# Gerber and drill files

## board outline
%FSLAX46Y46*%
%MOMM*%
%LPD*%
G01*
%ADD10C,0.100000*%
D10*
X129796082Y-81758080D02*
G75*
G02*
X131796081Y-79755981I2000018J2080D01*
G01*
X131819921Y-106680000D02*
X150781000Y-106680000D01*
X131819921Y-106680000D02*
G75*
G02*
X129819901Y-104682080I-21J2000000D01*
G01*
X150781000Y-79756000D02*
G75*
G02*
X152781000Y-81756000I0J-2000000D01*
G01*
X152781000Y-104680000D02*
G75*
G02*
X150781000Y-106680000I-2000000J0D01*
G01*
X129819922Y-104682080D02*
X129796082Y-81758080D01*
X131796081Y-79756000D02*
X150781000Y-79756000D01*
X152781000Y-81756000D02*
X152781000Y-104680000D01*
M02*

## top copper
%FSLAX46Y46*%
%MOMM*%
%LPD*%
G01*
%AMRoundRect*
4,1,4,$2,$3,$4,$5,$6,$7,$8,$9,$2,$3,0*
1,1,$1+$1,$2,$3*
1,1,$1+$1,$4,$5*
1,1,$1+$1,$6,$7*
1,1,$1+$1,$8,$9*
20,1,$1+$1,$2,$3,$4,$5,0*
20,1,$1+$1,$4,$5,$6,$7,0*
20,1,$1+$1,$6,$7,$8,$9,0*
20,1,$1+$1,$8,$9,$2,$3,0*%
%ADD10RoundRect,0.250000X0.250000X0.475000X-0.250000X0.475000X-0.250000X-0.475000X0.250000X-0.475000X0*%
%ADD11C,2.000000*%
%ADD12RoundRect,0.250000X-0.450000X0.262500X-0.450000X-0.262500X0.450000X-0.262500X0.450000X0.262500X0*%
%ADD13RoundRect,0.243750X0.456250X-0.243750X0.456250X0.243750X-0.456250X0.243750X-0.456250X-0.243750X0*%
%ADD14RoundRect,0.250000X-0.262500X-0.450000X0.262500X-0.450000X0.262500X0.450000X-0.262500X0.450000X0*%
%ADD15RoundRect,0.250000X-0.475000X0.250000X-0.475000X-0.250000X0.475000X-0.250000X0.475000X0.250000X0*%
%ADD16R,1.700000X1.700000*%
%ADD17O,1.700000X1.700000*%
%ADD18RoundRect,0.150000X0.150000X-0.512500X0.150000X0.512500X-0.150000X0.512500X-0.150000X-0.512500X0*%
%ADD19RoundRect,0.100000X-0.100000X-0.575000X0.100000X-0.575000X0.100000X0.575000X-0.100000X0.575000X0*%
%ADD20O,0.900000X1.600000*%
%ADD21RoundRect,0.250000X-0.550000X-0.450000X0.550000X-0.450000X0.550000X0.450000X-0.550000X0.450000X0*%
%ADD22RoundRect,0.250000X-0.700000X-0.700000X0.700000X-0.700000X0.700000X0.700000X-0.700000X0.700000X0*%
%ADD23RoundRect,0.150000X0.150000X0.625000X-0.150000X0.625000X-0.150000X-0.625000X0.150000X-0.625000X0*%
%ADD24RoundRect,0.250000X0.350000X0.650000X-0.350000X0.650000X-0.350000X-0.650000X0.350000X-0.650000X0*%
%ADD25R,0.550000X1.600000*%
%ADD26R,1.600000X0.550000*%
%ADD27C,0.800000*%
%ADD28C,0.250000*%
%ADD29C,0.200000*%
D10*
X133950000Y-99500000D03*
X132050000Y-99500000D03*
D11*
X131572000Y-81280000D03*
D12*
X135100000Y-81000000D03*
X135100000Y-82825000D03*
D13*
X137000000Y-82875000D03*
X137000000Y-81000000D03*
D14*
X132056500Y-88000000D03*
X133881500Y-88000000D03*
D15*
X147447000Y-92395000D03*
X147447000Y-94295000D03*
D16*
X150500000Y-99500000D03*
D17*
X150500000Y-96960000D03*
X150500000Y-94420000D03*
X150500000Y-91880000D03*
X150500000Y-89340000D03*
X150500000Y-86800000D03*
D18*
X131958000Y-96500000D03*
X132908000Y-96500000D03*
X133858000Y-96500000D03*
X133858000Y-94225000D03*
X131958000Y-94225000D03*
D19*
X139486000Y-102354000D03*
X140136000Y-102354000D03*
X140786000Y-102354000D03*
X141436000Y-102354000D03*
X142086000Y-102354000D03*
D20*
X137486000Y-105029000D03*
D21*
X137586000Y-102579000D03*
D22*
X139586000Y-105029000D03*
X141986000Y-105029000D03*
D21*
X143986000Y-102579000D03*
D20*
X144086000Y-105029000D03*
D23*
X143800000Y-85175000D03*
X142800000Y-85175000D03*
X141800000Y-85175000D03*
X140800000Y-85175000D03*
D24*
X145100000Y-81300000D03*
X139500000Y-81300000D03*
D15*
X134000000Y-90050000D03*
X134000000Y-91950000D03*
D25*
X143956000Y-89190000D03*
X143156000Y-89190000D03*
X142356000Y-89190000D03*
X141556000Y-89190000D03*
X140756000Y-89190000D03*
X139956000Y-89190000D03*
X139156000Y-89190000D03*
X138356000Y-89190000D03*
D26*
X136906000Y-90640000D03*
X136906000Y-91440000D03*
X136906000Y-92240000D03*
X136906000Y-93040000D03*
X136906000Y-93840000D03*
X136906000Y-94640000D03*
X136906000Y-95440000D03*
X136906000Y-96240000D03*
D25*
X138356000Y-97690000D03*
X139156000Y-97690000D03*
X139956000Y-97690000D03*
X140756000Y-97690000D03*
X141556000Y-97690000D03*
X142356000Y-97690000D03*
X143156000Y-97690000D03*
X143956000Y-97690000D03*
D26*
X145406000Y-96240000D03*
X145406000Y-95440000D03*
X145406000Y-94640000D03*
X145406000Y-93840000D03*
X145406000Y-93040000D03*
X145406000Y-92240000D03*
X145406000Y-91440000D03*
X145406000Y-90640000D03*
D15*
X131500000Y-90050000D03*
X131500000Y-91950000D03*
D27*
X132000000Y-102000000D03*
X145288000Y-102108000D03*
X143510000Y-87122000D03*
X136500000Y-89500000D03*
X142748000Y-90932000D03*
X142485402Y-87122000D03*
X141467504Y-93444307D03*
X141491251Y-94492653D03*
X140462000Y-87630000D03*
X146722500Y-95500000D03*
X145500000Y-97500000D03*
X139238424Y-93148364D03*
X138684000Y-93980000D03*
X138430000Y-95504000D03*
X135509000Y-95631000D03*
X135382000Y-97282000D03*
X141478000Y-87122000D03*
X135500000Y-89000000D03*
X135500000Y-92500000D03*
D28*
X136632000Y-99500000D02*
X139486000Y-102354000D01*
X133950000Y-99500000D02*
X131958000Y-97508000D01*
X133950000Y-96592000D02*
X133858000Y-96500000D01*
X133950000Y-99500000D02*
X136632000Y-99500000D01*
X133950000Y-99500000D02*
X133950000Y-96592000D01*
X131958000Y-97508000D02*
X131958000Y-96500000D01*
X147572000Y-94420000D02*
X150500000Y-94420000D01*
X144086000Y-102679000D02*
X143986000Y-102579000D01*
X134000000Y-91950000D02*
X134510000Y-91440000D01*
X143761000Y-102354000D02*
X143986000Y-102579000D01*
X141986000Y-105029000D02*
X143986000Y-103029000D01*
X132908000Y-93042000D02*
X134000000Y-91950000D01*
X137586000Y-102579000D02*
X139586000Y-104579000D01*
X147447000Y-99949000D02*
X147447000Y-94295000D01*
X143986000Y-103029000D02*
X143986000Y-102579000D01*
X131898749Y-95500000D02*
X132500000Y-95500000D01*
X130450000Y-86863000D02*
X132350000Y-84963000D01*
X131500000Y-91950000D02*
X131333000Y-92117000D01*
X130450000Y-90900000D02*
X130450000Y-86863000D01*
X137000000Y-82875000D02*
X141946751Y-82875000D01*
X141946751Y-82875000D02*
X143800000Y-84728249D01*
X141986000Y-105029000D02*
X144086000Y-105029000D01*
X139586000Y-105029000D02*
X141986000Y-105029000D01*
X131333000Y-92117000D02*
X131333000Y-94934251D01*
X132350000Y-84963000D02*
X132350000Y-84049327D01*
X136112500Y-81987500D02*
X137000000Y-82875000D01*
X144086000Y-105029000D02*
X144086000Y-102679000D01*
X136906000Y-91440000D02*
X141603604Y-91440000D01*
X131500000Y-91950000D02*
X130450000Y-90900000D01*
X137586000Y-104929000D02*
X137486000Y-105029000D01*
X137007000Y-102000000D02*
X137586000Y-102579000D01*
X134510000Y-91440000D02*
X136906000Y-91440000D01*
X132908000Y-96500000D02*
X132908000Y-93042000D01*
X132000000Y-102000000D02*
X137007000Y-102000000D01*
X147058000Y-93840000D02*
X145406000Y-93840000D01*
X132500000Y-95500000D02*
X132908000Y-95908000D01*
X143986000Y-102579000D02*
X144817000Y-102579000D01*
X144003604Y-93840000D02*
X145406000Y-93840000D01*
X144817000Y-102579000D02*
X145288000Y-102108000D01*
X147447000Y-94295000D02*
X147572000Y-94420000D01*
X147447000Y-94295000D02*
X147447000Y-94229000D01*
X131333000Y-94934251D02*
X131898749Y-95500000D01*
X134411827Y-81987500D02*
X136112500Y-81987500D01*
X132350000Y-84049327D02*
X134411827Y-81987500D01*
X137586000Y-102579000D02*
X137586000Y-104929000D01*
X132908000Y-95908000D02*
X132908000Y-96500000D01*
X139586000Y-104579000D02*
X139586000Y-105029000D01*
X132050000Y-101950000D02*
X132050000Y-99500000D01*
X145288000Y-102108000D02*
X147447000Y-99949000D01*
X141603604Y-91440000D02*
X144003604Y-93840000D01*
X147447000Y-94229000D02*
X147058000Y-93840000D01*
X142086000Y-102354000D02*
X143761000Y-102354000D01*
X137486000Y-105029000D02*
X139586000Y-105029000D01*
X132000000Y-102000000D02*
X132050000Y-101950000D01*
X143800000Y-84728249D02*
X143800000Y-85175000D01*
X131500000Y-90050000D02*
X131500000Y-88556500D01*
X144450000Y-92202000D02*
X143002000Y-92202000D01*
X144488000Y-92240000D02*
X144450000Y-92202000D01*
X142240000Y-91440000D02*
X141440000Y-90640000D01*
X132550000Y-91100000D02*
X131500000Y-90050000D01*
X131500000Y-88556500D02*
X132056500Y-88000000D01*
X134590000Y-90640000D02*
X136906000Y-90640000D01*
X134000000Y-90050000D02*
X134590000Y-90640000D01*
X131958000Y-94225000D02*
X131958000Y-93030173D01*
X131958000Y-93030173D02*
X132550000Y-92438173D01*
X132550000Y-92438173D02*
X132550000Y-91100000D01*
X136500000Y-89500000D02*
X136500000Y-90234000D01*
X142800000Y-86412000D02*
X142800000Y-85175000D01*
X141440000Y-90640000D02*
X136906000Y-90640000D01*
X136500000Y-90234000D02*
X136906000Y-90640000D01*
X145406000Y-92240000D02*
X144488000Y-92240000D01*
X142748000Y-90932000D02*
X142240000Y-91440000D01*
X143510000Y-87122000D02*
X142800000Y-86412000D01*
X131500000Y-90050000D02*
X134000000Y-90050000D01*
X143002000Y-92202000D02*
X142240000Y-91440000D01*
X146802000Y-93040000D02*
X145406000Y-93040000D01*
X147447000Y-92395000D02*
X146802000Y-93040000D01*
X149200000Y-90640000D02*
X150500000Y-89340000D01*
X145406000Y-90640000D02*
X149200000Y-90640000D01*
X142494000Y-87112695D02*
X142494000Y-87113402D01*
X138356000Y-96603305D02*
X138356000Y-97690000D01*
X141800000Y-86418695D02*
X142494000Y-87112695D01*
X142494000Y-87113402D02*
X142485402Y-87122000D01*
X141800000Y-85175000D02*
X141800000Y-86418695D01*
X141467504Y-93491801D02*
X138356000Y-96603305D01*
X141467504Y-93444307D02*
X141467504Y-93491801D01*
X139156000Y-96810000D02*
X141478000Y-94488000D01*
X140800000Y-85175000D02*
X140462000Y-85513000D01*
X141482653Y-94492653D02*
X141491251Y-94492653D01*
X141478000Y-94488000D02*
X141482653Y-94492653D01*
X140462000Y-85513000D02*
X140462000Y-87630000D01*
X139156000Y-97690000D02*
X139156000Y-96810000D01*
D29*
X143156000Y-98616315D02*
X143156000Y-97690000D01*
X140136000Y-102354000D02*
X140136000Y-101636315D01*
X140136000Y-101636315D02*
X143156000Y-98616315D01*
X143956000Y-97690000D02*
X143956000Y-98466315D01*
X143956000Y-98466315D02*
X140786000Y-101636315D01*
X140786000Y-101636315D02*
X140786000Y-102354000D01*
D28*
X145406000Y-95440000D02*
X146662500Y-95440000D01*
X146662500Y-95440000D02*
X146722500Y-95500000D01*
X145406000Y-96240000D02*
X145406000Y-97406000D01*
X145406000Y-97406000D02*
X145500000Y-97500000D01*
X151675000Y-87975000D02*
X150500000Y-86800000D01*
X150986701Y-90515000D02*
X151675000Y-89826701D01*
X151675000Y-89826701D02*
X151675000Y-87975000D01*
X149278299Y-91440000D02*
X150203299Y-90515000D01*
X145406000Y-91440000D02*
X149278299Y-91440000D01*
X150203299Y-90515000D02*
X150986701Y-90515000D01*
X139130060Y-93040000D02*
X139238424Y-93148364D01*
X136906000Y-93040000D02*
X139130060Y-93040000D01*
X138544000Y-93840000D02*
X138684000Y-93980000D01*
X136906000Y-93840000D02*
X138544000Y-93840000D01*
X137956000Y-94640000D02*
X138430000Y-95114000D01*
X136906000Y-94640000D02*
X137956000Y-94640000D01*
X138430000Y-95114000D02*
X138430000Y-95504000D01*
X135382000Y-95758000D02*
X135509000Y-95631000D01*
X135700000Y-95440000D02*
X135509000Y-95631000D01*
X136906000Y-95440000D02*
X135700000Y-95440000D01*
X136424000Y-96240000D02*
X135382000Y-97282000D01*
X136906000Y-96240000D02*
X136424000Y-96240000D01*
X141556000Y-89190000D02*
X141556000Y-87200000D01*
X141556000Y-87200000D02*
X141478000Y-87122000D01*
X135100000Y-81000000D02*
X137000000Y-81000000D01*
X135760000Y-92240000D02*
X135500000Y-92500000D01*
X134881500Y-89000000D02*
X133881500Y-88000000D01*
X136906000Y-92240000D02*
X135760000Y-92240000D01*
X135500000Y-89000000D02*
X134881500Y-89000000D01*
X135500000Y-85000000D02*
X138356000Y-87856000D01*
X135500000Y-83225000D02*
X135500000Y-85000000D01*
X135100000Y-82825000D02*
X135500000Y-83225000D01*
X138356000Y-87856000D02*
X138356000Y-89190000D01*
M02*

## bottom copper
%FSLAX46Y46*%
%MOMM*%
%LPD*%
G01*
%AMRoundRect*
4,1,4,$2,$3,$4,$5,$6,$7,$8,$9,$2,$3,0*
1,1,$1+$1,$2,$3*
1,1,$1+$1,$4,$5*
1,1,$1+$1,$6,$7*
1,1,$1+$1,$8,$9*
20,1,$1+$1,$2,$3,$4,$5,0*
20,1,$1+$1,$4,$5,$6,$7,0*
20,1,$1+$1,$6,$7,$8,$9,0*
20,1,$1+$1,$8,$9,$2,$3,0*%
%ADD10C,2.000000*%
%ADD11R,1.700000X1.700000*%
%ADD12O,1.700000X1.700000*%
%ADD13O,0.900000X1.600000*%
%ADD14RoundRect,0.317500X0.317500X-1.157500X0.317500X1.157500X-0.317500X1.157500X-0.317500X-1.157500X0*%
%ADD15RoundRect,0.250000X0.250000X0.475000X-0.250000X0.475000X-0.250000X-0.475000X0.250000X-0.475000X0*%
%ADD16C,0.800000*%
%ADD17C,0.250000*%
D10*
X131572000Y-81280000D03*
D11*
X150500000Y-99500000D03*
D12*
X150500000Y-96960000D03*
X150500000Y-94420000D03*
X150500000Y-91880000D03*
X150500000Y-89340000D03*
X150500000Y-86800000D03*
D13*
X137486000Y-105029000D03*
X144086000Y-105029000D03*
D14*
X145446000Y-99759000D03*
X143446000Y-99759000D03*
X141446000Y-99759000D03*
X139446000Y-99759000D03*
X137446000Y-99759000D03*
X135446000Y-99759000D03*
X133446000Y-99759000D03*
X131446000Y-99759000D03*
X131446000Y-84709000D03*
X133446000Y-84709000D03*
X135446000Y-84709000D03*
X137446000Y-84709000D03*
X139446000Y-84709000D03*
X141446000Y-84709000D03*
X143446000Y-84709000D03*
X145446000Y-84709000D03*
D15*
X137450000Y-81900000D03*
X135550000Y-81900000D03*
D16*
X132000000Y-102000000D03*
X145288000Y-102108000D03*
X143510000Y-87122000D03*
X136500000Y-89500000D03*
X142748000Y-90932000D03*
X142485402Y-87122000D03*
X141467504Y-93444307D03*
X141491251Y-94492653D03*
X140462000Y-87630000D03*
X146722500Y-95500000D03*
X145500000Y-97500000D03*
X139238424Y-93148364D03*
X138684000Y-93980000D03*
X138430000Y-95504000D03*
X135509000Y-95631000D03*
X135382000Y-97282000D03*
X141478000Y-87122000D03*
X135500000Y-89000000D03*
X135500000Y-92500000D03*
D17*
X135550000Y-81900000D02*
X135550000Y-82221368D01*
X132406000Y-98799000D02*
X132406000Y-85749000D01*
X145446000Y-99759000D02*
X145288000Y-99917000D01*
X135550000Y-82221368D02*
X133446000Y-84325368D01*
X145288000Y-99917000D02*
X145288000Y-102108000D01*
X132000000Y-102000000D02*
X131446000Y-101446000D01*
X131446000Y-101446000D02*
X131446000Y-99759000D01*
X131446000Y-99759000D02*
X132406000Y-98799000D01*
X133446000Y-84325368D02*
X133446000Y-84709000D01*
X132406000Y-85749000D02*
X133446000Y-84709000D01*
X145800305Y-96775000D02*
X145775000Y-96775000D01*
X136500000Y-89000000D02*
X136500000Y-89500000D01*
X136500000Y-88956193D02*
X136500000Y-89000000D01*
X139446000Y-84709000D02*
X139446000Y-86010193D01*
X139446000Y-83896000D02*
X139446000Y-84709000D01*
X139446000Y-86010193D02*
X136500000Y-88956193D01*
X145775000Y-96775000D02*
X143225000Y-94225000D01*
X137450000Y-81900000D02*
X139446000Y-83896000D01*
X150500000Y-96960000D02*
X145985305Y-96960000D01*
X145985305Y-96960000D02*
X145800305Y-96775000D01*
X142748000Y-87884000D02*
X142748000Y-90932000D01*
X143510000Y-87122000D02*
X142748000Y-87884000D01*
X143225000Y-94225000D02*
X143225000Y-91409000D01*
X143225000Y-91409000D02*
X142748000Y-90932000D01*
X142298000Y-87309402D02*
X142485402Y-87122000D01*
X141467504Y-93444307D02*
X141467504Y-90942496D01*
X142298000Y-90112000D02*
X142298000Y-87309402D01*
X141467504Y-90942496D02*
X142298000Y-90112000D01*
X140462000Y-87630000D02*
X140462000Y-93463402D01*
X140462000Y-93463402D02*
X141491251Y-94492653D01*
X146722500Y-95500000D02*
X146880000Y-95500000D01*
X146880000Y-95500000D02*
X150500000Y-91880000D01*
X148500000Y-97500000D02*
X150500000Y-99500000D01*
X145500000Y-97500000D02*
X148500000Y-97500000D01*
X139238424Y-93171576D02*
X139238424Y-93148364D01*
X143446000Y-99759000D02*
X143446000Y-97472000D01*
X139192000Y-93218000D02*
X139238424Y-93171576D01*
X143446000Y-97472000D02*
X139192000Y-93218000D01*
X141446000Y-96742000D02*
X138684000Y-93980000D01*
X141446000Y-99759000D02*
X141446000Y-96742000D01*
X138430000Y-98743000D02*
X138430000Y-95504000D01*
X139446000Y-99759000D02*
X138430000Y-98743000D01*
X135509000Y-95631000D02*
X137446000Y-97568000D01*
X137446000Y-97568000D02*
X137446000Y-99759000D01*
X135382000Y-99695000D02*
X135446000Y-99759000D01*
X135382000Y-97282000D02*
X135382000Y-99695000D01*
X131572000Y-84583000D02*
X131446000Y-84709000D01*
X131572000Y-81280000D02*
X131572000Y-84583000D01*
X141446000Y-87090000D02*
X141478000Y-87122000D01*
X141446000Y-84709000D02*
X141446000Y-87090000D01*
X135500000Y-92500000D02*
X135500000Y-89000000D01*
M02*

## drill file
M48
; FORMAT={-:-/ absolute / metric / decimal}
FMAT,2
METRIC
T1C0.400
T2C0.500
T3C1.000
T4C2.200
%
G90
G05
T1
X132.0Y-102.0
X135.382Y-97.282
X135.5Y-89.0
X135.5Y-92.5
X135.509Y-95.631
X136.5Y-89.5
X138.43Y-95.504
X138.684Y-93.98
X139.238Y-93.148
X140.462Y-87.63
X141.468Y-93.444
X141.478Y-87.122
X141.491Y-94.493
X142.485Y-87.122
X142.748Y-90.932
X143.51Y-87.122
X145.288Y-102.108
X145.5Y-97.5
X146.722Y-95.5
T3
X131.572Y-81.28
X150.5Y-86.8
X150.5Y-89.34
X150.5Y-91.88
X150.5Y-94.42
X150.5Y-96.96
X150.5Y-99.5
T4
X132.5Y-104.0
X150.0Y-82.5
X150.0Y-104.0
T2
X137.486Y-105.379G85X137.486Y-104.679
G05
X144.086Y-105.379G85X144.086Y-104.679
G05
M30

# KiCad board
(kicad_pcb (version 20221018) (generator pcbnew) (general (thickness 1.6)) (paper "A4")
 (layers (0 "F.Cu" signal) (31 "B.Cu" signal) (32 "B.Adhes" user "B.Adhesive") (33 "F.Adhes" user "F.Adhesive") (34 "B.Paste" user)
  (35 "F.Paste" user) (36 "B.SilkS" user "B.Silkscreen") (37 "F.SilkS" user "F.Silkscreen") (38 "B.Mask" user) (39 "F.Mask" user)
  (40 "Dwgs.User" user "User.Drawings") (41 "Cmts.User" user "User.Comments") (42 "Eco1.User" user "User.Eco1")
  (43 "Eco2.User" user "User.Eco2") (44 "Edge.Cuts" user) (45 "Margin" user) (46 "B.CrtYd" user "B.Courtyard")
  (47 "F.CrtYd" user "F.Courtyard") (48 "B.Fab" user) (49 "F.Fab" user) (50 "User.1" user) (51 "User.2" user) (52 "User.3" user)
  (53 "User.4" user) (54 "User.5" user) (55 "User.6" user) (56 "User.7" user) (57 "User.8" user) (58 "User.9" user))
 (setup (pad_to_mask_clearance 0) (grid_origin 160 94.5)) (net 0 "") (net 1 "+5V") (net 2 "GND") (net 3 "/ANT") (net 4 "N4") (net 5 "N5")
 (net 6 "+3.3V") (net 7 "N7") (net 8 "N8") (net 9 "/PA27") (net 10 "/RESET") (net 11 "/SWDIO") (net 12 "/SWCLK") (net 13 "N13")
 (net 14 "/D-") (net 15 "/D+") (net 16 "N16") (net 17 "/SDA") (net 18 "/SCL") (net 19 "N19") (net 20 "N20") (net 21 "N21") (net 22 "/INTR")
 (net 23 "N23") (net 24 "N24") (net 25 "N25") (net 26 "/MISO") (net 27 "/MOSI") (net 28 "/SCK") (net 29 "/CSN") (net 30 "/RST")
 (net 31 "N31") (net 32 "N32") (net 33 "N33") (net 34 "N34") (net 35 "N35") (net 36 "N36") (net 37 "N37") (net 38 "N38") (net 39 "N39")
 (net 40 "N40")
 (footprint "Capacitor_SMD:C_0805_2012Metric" (layer "F.Cu") (at 133 99.5 180)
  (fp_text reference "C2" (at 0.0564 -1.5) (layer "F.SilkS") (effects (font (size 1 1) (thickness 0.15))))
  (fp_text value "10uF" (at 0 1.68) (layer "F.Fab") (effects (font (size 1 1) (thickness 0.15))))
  (pad "1" smd roundrect (at -0.95 0 180) (size 1 1.45) (layers "F.Cu" "F.Paste" "F.Mask") (roundrect_rratio 0.25) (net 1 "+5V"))
  (pad "2" smd roundrect (at 0.95 0 180) (size 1 1.45) (layers "F.Cu" "F.Paste" "F.Mask") (roundrect_rratio 0.25) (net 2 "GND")))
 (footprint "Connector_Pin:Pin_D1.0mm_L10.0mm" (layer "F.Cu") (at 131.572 81.28)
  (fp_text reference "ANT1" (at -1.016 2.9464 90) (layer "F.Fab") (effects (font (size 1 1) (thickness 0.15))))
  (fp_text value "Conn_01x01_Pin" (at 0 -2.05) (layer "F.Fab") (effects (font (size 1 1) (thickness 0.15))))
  (pad "1" thru_hole circle (at 0 0) (size 2 2) (drill 1) (layers "*.Cu" "*.Mask") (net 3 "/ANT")))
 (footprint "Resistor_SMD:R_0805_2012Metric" (layer "F.Cu") (at 135.1 81.9125 -90)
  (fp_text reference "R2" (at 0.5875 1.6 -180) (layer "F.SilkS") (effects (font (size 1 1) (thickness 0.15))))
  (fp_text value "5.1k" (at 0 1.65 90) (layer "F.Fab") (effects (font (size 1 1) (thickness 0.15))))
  (pad "1" smd roundrect (at -0.9125 0 270) (size 1.025 1.4) (layers "F.Cu" "F.Paste" "F.Mask") (roundrect_rratio 0.243902) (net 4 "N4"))
  (pad "2" smd roundrect (at 0.9125 0 270) (size 1.025 1.4) (layers "F.Cu" "F.Paste" "F.Mask") (roundrect_rratio 0.243902) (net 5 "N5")))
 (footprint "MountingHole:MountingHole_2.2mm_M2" (layer "F.Cu") (at 150 104)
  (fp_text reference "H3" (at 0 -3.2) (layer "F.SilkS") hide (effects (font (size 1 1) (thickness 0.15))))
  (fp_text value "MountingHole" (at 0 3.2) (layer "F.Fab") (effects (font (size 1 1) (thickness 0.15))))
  (pad "" np_thru_hole circle (at 0 0) (size 2.2 2.2) (drill 2.2) (layers "*.Cu" "*.Mask")))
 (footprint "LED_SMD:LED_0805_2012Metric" (layer "F.Cu") (at 137 81.9375 90)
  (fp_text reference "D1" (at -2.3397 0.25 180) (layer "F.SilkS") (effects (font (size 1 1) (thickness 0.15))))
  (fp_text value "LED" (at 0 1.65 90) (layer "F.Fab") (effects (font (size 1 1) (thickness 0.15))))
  (pad "1" smd roundrect (at -0.9375 0 90) (size 0.975 1.4) (layers "F.Cu" "F.Paste" "F.Mask") (roundrect_rratio 0.25) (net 2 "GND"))
  (pad "2" smd roundrect (at 0.9375 0 90) (size 0.975 1.4) (layers "F.Cu" "F.Paste" "F.Mask") (roundrect_rratio 0.25) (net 4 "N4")))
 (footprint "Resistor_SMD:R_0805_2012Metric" (layer "F.Cu") (at 132.969 88)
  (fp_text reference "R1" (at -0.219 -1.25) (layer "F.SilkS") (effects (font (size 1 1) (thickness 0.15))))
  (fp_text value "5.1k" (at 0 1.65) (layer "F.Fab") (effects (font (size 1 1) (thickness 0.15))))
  (pad "1" smd roundrect (at -0.9125 0) (size 1.025 1.4) (layers "F.Cu" "F.Paste" "F.Mask") (roundrect_rratio 0.243902) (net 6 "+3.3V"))
  (pad "2" smd roundrect (at 0.9125 0) (size 1.025 1.4) (layers "F.Cu" "F.Paste" "F.Mask") (roundrect_rratio 0.243902) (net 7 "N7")))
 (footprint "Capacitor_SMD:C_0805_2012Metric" (layer "F.Cu") (at 147.447 93.345 -90)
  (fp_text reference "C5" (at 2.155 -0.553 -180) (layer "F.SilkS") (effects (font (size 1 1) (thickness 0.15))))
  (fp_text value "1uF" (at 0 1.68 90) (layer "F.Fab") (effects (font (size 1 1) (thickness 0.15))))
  (pad "1" smd roundrect (at -0.95 0 270) (size 1 1.45) (layers "F.Cu" "F.Paste" "F.Mask") (roundrect_rratio 0.25) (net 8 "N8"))
  (pad "2" smd roundrect (at 0.95 0 270) (size 1 1.45) (layers "F.Cu" "F.Paste" "F.Mask") (roundrect_rratio 0.25) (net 2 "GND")))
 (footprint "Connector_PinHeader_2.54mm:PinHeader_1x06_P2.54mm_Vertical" (layer "F.Cu") (at 150.5 99.5 180)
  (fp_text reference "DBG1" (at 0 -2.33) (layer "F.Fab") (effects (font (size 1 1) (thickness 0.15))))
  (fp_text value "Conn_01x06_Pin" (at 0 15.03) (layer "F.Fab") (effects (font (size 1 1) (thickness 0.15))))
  (pad "1" thru_hole rect (at 0 0 180) (size 1.7 1.7) (drill 1) (layers "*.Cu" "*.Mask") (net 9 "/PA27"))
  (pad "2" thru_hole oval (at 0 2.54 180) (size 1.7 1.7) (drill 1) (layers "*.Cu" "*.Mask") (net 6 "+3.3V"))
  (pad "3" thru_hole oval (at 0 5.08 180) (size 1.7 1.7) (drill 1) (layers "*.Cu" "*.Mask") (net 2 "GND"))
  (pad "4" thru_hole oval (at 0 7.62 180) (size 1.7 1.7) (drill 1) (layers "*.Cu" "*.Mask") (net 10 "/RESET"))
  (pad "5" thru_hole oval (at 0 10.16 180) (size 1.7 1.7) (drill 1) (layers "*.Cu" "*.Mask") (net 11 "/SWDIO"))
  (pad "6" thru_hole oval (at 0 12.7 180) (size 1.7 1.7) (drill 1) (layers "*.Cu" "*.Mask") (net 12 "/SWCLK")))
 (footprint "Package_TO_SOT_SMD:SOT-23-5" (layer "F.Cu") (at 132.908 95.3625 90)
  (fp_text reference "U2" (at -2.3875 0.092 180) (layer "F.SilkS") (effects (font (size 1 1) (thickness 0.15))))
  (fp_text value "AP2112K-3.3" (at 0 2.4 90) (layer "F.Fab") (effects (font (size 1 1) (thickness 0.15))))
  (pad "1" smd roundrect (at -1.1375 -0.95 90) (size 1.325 0.6) (layers "F.Cu" "F.Paste" "F.Mask") (roundrect_rratio 0.25) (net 1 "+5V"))
  (pad "2" smd roundrect (at -1.1375 0 90) (size 1.325 0.6) (layers "F.Cu" "F.Paste" "F.Mask") (roundrect_rratio 0.25) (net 2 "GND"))
  (pad "3" smd roundrect (at -1.1375 0.95 90) (size 1.325 0.6) (layers "F.Cu" "F.Paste" "F.Mask") (roundrect_rratio 0.25) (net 1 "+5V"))
  (pad "4" smd roundrect (at 1.1375 0.95 90) (size 1.325 0.6) (layers "F.Cu" "F.Paste" "F.Mask") (roundrect_rratio 0.25) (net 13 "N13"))
  (pad "5" smd roundrect (at 1.1375 -0.95 90) (size 1.325 0.6) (layers "F.Cu" "F.Paste" "F.Mask") (roundrect_rratio 0.25) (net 6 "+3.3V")))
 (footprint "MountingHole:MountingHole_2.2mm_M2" (layer "F.Cu") (at 150 82.5)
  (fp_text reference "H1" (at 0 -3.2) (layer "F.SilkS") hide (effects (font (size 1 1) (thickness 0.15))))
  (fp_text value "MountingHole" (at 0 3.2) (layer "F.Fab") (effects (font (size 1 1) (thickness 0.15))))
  (pad "" np_thru_hole circle (at 0 0) (size 2.2 2.2) (drill 2.2) (layers "*.Cu" "*.Mask")))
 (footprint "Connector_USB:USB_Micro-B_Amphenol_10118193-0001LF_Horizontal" (layer "F.Cu") (at 140.786 105.029)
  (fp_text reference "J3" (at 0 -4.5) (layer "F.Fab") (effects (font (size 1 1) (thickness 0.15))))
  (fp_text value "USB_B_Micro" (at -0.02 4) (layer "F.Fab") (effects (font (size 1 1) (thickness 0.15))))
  (pad "1" smd roundrect (at -1.3 -2.675) (size 0.4 1.35) (layers "F.Cu" "F.Paste" "F.Mask") (roundrect_rratio 0.25) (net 1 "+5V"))
  (pad "2" smd roundrect (at -0.65 -2.675) (size 0.4 1.35) (layers "F.Cu" "F.Paste" "F.Mask") (roundrect_rratio 0.25) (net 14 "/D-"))
  (pad "3" smd roundrect (at 0 -2.675) (size 0.4 1.35) (layers "F.Cu" "F.Paste" "F.Mask") (roundrect_rratio 0.25) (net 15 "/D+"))
  (pad "4" smd roundrect (at 0.65 -2.675) (size 0.4 1.35) (layers "F.Cu" "F.Paste" "F.Mask") (roundrect_rratio 0.25) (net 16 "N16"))
  (pad "5" smd roundrect (at 1.3 -2.675) (size 0.4 1.35) (layers "F.Cu" "F.Paste" "F.Mask") (roundrect_rratio 0.25) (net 2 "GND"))
  (pad "6" thru_hole oval (at -3.3 0 90) (size 1.6 0.9) (drill oval 1.2 0.5) (layers "*.Cu" "*.Mask" "F.Paste") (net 2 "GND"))
  (pad "6" smd roundrect (at -3.2 -2.45) (size 1.6 1.4) (layers "F.Cu" "F.Paste" "F.Mask") (roundrect_rratio 0.1785714286) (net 2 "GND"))
  (pad "6" smd roundrect (at -1.2 0) (size 1.9 1.9) (layers "F.Cu" "F.Paste" "F.Mask") (roundrect_rratio 0.1315789474) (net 2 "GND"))
  (pad "6" smd roundrect (at 1.2 0) (size 1.9 1.9) (layers "F.Cu" "F.Paste" "F.Mask") (roundrect_rratio 0.1315789474) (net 2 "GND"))
  (pad "6" smd roundrect (at 3.2 -2.45) (size 1.6 1.4) (layers "F.Cu" "F.Paste" "F.Mask") (roundrect_rratio 0.1785714286) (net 2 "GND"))
  (pad "6" thru_hole oval (at 3.3 0 90) (size 1.6 0.9) (drill oval 1.2 0.5) (layers "*.Cu" "*.Mask" "F.Paste") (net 2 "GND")))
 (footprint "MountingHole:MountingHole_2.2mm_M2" (layer "F.Cu") (at 132.5 104)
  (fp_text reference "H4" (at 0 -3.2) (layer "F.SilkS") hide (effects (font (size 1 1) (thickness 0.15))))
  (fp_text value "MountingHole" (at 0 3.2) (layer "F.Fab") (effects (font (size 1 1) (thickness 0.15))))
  (pad "" np_thru_hole circle (at 0 0) (size 2.2 2.2) (drill 2.2) (layers "*.Cu" "*.Mask")))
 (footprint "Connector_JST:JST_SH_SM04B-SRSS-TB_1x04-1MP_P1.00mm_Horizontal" (layer "F.Cu") (at 142.3 83.175 180)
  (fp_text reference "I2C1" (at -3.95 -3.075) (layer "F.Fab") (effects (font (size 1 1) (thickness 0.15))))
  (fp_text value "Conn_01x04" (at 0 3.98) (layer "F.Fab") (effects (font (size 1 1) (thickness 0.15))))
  (pad "1" smd roundrect (at -1.5 -2 180) (size 0.6 1.55) (layers "F.Cu" "F.Paste" "F.Mask") (roundrect_rratio 0.25) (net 2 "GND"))
  (pad "2" smd roundrect (at -0.5 -2 180) (size 0.6 1.55) (layers "F.Cu" "F.Paste" "F.Mask") (roundrect_rratio 0.25) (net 6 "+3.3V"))
  (pad "3" smd roundrect (at 0.5 -2 180) (size 0.6 1.55) (layers "F.Cu" "F.Paste" "F.Mask") (roundrect_rratio 0.25) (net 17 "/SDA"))
  (pad "4" smd roundrect (at 1.5 -2 180) (size 0.6 1.55) (layers "F.Cu" "F.Paste" "F.Mask") (roundrect_rratio 0.25) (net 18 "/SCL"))
  (pad "MP" smd roundrect (at -2.8 1.875 180) (size 1.2 1.8) (layers "F.Cu" "F.Paste" "F.Mask") (roundrect_rratio 0.208333))
  (pad "MP" smd roundrect (at 2.8 1.875 180) (size 1.2 1.8) (layers "F.Cu" "F.Paste" "F.Mask") (roundrect_rratio 0.208333)))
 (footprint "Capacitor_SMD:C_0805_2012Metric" (layer "F.Cu") (at 134 91 -90)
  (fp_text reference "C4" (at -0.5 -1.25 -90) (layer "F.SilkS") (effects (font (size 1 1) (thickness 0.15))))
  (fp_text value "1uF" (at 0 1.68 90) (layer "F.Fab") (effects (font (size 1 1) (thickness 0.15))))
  (pad "1" smd roundrect (at -0.95 0 270) (size 1 1.45) (layers "F.Cu" "F.Paste" "F.Mask") (roundrect_rratio 0.25) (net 6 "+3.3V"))
  (pad "2" smd roundrect (at 0.95 0 270) (size 1 1.45) (layers "F.Cu" "F.Paste" "F.Mask") (roundrect_rratio 0.25) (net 2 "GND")))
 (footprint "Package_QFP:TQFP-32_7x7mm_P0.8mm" (layer "F.Cu") (at 141.156 93.44 -90)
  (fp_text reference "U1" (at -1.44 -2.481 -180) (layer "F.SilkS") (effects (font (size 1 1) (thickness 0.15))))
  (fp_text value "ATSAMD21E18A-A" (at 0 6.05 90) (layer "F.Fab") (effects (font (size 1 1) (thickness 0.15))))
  (pad "1" smd rect (at -4.25 -2.8 270) (size 1.6 0.55) (layers "F.Cu" "F.Paste" "F.Mask") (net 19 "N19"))
  (pad "2" smd rect (at -4.25 -2 270) (size 1.6 0.55) (layers "F.Cu" "F.Paste" "F.Mask") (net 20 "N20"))
  (pad "3" smd rect (at -4.25 -1.2 270) (size 1.6 0.55) (layers "F.Cu" "F.Paste" "F.Mask") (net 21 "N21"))
  (pad "4" smd rect (at -4.25 -0.4 270) (size 1.6 0.55) (layers "F.Cu" "F.Paste" "F.Mask") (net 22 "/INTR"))
  (pad "5" smd rect (at -4.25 0.4 270) (size 1.6 0.55) (layers "F.Cu" "F.Paste" "F.Mask") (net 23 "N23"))
  (pad "6" smd rect (at -4.25 1.2 270) (size 1.6 0.55) (layers "F.Cu" "F.Paste" "F.Mask") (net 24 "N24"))
  (pad "7" smd rect (at -4.25 2 270) (size 1.6 0.55) (layers "F.Cu" "F.Paste" "F.Mask") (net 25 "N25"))
  (pad "8" smd rect (at -4.25 2.8 270) (size 1.6 0.55) (layers "F.Cu" "F.Paste" "F.Mask") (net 5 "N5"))
  (pad "9" smd rect (at -2.8 4.25) (size 1.6 0.55) (layers "F.Cu" "F.Paste" "F.Mask") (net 6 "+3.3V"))
  (pad "10" smd rect (at -2 4.25) (size 1.6 0.55) (layers "F.Cu" "F.Paste" "F.Mask") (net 2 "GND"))
  (pad "11" smd rect (at -1.2 4.25) (size 1.6 0.55) (layers "F.Cu" "F.Paste" "F.Mask") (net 7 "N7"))
  (pad "12" smd rect (at -0.4 4.25) (size 1.6 0.55) (layers "F.Cu" "F.Paste" "F.Mask") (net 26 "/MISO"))
  (pad "13" smd rect (at 0.4 4.25) (size 1.6 0.55) (layers "F.Cu" "F.Paste" "F.Mask") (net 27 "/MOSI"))
  (pad "14" smd rect (at 1.2 4.25) (size 1.6 0.55) (layers "F.Cu" "F.Paste" "F.Mask") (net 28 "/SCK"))
  (pad "15" smd rect (at 2 4.25) (size 1.6 0.55) (layers "F.Cu" "F.Paste" "F.Mask") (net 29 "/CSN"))
  (pad "16" smd rect (at 2.8 4.25) (size 1.6 0.55) (layers "F.Cu" "F.Paste" "F.Mask") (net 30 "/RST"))
  (pad "17" smd rect (at 4.25 2.8 270) (size 1.6 0.55) (layers "F.Cu" "F.Paste" "F.Mask") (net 17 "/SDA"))
  (pad "18" smd rect (at 4.25 2 270) (size 1.6 0.55) (layers "F.Cu" "F.Paste" "F.Mask") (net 18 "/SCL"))
  (pad "19" smd rect (at 4.25 1.2 270) (size 1.6 0.55) (layers "F.Cu" "F.Paste" "F.Mask") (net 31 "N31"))
  (pad "20" smd rect (at 4.25 0.4 270) (size 1.6 0.55) (layers "F.Cu" "F.Paste" "F.Mask") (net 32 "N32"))
  (pad "21" smd rect (at 4.25 -0.4 270) (size 1.6 0.55) (layers "F.Cu" "F.Paste" "F.Mask") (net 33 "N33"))
  (pad "22" smd rect (at 4.25 -1.2 270) (size 1.6 0.55) (layers "F.Cu" "F.Paste" "F.Mask") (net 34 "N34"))
  (pad "23" smd rect (at 4.25 -2 270) (size 1.6 0.55) (layers "F.Cu" "F.Paste" "F.Mask") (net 14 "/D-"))
  (pad "24" smd rect (at 4.25 -2.8 270) (size 1.6 0.55) (layers "F.Cu" "F.Paste" "F.Mask") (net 15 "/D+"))
  (pad "25" smd rect (at 2.8 -4.25) (size 1.6 0.55) (layers "F.Cu" "F.Paste" "F.Mask") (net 9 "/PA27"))
  (pad "26" smd rect (at 2 -4.25) (size 1.6 0.55) (layers "F.Cu" "F.Paste" "F.Mask") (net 10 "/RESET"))
  (pad "27" smd rect (at 1.2 -4.25) (size 1.6 0.55) (layers "F.Cu" "F.Paste" "F.Mask") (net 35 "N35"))
  (pad "28" smd rect (at 0.4 -4.25) (size 1.6 0.55) (layers "F.Cu" "F.Paste" "F.Mask") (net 2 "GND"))
  (pad "29" smd rect (at -0.4 -4.25) (size 1.6 0.55) (layers "F.Cu" "F.Paste" "F.Mask") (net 8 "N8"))
  (pad "30" smd rect (at -1.2 -4.25) (size 1.6 0.55) (layers "F.Cu" "F.Paste" "F.Mask") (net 6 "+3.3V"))
  (pad "31" smd rect (at -2 -4.25) (size 1.6 0.55) (layers "F.Cu" "F.Paste" "F.Mask") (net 12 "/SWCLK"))
  (pad "32" smd rect (at -2.8 -4.25) (size 1.6 0.55) (layers "F.Cu" "F.Paste" "F.Mask") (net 11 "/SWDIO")))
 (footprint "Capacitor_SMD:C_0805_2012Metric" (layer "F.Cu") (at 131.5 91 -90)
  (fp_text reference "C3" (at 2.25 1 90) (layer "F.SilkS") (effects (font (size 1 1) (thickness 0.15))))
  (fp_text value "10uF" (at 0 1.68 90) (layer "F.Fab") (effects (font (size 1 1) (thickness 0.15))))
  (pad "1" smd roundrect (at -0.95 0 270) (size 1 1.45) (layers "F.Cu" "F.Paste" "F.Mask") (roundrect_rratio 0.25) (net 6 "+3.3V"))
  (pad "2" smd roundrect (at 0.95 0 270) (size 1 1.45) (layers "F.Cu" "F.Paste" "F.Mask") (roundrect_rratio 0.25) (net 2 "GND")))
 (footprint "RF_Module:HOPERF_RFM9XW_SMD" (layer "B.Cu") (at 138.446 92.234 90)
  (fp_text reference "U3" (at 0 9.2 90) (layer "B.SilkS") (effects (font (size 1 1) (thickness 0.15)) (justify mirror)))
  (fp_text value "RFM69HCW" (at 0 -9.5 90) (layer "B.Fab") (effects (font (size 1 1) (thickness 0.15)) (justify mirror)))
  (pad "1" smd roundrect (at -7.525 7 90) (size 2.95 1.27) (layers "B.Cu" "B.Paste" "B.Mask") (roundrect_rratio 0.25) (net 2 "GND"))
  (pad "2" smd roundrect (at -7.525 5 90) (size 2.95 1.27) (layers "B.Cu" "B.Paste" "B.Mask") (roundrect_rratio 0.25) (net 26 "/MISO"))
  (pad "3" smd roundrect (at -7.525 3 90) (size 2.95 1.27) (layers "B.Cu" "B.Paste" "B.Mask") (roundrect_rratio 0.25) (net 27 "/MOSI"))
  (pad "4" smd roundrect (at -7.525 1 90) (size 2.95 1.27) (layers "B.Cu" "B.Paste" "B.Mask") (roundrect_rratio 0.25) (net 28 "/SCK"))
  (pad "5" smd roundrect (at -7.525 -1 90) (size 2.95 1.27) (layers "B.Cu" "B.Paste" "B.Mask") (roundrect_rratio 0.25) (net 29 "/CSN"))
  (pad "6" smd roundrect (at -7.525 -3 90) (size 2.95 1.27) (layers "B.Cu" "B.Paste" "B.Mask") (roundrect_rratio 0.25) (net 30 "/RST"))
  (pad "7" smd roundrect (at -7.525 -5 90) (size 2.95 1.27) (layers "B.Cu" "B.Paste" "B.Mask") (roundrect_rratio 0.25) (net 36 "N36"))
  (pad "8" smd roundrect (at -7.525 -7 90) (size 2.95 1.27) (layers "B.Cu" "B.Paste" "B.Mask") (roundrect_rratio 0.25) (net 2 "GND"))
  (pad "9" smd roundrect (at 7.525 -7 90) (size 2.95 1.27) (layers "B.Cu" "B.Paste" "B.Mask") (roundrect_rratio 0.25) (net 3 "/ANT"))
  (pad "10" smd roundrect (at 7.525 -5 90) (size 2.95 1.27) (layers "B.Cu" "B.Paste" "B.Mask") (roundrect_rratio 0.25) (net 2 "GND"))
  (pad "11" smd roundrect (at 7.525 -3 90) (size 2.95 1.27) (layers "B.Cu" "B.Paste" "B.Mask") (roundrect_rratio 0.25) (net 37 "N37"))
  (pad "12" smd roundrect (at 7.525 -1 90) (size 2.95 1.27) (layers "B.Cu" "B.Paste" "B.Mask") (roundrect_rratio 0.25) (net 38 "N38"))
  (pad "13" smd roundrect (at 7.525 1 90) (size 2.95 1.27) (layers "B.Cu" "B.Paste" "B.Mask") (roundrect_rratio 0.25) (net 6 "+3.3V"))
  (pad "14" smd roundrect (at 7.525 3 90) (size 2.95 1.27) (layers "B.Cu" "B.Paste" "B.Mask") (roundrect_rratio 0.25) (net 22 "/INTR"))
  (pad "15" smd roundrect (at 7.525 5 90) (size 2.95 1.27) (layers "B.Cu" "B.Paste" "B.Mask") (roundrect_rratio 0.25) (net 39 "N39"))
  (pad "16" smd roundrect (at 7.525 7 90) (size 2.95 1.27) (layers "B.Cu" "B.Paste" "B.Mask") (roundrect_rratio 0.25) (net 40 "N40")))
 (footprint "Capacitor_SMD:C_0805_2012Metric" (layer "B.Cu") (at 136.5 81.9 180)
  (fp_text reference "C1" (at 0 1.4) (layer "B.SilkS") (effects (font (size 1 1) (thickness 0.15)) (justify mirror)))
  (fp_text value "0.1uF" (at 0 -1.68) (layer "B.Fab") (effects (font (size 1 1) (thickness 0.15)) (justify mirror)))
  (pad "1" smd roundrect (at -0.95 0 180) (size 1 1.45) (layers "B.Cu" "B.Paste" "B.Mask") (roundrect_rratio 0.25) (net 6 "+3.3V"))
  (pad "2" smd roundrect (at 0.95 0 180) (size 1 1.45) (layers "B.Cu" "B.Paste" "B.Mask") (roundrect_rratio 0.25) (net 2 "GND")))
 (gr_arc (start 129.796082 81.75808) (mid 130.381132 80.342522) (end 131.796081 79.756) (stroke (width 0.1) (type default))
  (layer "Edge.Cuts"))
 (gr_line (start 131.819921 106.68) (end 150.781 106.68) (stroke (width 0.1) (type default)) (layer "Edge.Cuts"))
 (gr_arc (start 131.819921 106.68) (mid 130.406443 106.094949) (end 129.819922 104.68208) (stroke (width 0.1) (type default))
  (layer "Edge.Cuts"))
 (gr_arc (start 150.781 79.756) (mid 152.195214 80.341786) (end 152.781 81.756) (stroke (width 0.1) (type default)) (layer "Edge.Cuts"))
 (gr_arc (start 152.781 104.68) (mid 152.195214 106.094214) (end 150.781 106.68) (stroke (width 0.1) (type default)) (layer "Edge.Cuts"))
 (gr_line (start 129.819922 104.68208) (end 129.796082 81.75808) (stroke (width 0.1) (type default)) (layer "Edge.Cuts"))
 (gr_line (start 131.796081 79.756) (end 150.781 79.756) (stroke (width 0.1) (type default)) (layer "Edge.Cuts"))
 (gr_line (start 152.781 81.756) (end 152.781 104.68) (stroke (width 0.1) (type default)) (layer "Edge.Cuts"))
 (segment (start 136.632 99.5) (end 139.486 102.354) (width 0.25) (layer "F.Cu") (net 1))
 (segment (start 133.95 99.5) (end 131.958 97.508) (width 0.25) (layer "F.Cu") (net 1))
 (segment (start 133.95 96.592) (end 133.858 96.5) (width 0.25) (layer "F.Cu") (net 1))
 (segment (start 133.95 99.5) (end 136.632 99.5) (width 0.25) (layer "F.Cu") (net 1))
 (segment (start 133.95 99.5) (end 133.95 96.592) (width 0.25) (layer "F.Cu") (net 1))
 (segment (start 131.958 97.508) (end 131.958 96.5) (width 0.25) (layer "F.Cu") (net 1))
 (segment (start 147.572 94.42) (end 150.5 94.42) (width 0.25) (layer "F.Cu") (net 2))
 (segment (start 144.086 102.679) (end 143.986 102.579) (width 0.25) (layer "F.Cu") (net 2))
 (segment (start 134 91.95) (end 134.51 91.44) (width 0.25) (layer "F.Cu") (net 2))
 (segment (start 143.761 102.354) (end 143.986 102.579) (width 0.25) (layer "F.Cu") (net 2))
 (segment (start 141.986 105.029) (end 143.986 103.029) (width 0.25) (layer "F.Cu") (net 2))
 (segment (start 132.908 93.042) (end 134 91.95) (width 0.25) (layer "F.Cu") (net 2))
 (segment (start 137.586 102.579) (end 139.586 104.579) (width 0.25) (layer "F.Cu") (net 2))
 (segment (start 147.447 99.949) (end 147.447 94.295) (width 0.25) (layer "F.Cu") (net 2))
 (segment (start 143.986 103.029) (end 143.986 102.579) (width 0.25) (layer "F.Cu") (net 2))
 (segment (start 131.898749 95.5) (end 132.5 95.5) (width 0.25) (layer "F.Cu") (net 2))
 (segment (start 130.45 86.863) (end 132.35 84.963) (width 0.25) (layer "F.Cu") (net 2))
 (segment (start 131.5 91.95) (end 131.333 92.117) (width 0.25) (layer "F.Cu") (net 2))
 (segment (start 130.45 90.9) (end 130.45 86.863) (width 0.25) (layer "F.Cu") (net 2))
 (segment (start 137 82.875) (end 141.946751 82.875) (width 0.25) (layer "F.Cu") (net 2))
 (segment (start 141.946751 82.875) (end 143.8 84.728249) (width 0.25) (layer "F.Cu") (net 2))
 (segment (start 141.986 105.029) (end 144.086 105.029) (width 0.25) (layer "F.Cu") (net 2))
 (segment (start 139.586 105.029) (end 141.986 105.029) (width 0.25) (layer "F.Cu") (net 2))
 (segment (start 131.333 92.117) (end 131.333 94.934251) (width 0.25) (layer "F.Cu") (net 2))
 (segment (start 132.35 84.963) (end 132.35 84.049327) (width 0.25) (layer "F.Cu") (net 2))
 (segment (start 136.1125 81.9875) (end 137 82.875) (width 0.25) (layer "F.Cu") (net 2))
 (segment (start 144.086 105.029) (end 144.086 102.679) (width 0.25) (layer "F.Cu") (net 2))
 (segment (start 136.906 91.44) (end 141.603604 91.44) (width 0.25) (layer "F.Cu") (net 2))
 (segment (start 131.5 91.95) (end 130.45 90.9) (width 0.25) (layer "F.Cu") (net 2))
 (segment (start 137.586 104.929) (end 137.486 105.029) (width 0.25) (layer "F.Cu") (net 2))
 (segment (start 137.007 102) (end 137.586 102.579) (width 0.25) (layer "F.Cu") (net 2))
 (segment (start 134.51 91.44) (end 136.906 91.44) (width 0.25) (layer "F.Cu") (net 2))
 (segment (start 132.908 96.5) (end 132.908 93.042) (width 0.25) (layer "F.Cu") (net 2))
 (segment (start 132 102) (end 137.007 102) (width 0.25) (layer "F.Cu") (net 2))
 (segment (start 147.058 93.84) (end 145.406 93.84) (width 0.25) (layer "F.Cu") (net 2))
 (segment (start 132.5 95.5) (end 132.908 95.908) (width 0.25) (layer "F.Cu") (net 2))
 (segment (start 143.986 102.579) (end 144.817 102.579) (width 0.25) (layer "F.Cu") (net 2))
 (segment (start 144.003604 93.84) (end 145.406 93.84) (width 0.25) (layer "F.Cu") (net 2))
 (segment (start 144.817 102.579) (end 145.288 102.108) (width 0.25) (layer "F.Cu") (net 2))
 (segment (start 147.447 94.295) (end 147.572 94.42) (width 0.25) (layer "F.Cu") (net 2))
 (segment (start 147.447 94.295) (end 147.447 94.229) (width 0.25) (layer "F.Cu") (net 2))
 (segment (start 131.333 94.934251) (end 131.898749 95.5) (width 0.25) (layer "F.Cu") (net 2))
 (segment (start 134.411827 81.9875) (end 136.1125 81.9875) (width 0.25) (layer "F.Cu") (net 2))
 (segment (start 132.35 84.049327) (end 134.411827 81.9875) (width 0.25) (layer "F.Cu") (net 2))
 (segment (start 137.586 102.579) (end 137.586 104.929) (width 0.25) (layer "F.Cu") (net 2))
 (segment (start 132.908 95.908) (end 132.908 96.5) (width 0.25) (layer "F.Cu") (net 2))
 (segment (start 139.586 104.579) (end 139.586 105.029) (width 0.25) (layer "F.Cu") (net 2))
 (segment (start 132.05 101.95) (end 132.05 99.5) (width 0.25) (layer "F.Cu") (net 2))
 (segment (start 145.288 102.108) (end 147.447 99.949) (width 0.25) (layer "F.Cu") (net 2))
 (segment (start 141.603604 91.44) (end 144.003604 93.84) (width 0.25) (layer "F.Cu") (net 2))
 (segment (start 147.447 94.229) (end 147.058 93.84) (width 0.25) (layer "F.Cu") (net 2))
 (segment (start 142.086 102.354) (end 143.761 102.354) (width 0.25) (layer "F.Cu") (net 2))
 (segment (start 137.486 105.029) (end 139.586 105.029) (width 0.25) (layer "F.Cu") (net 2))
 (segment (start 132 102) (end 132.05 101.95) (width 0.25) (layer "F.Cu") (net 2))
 (segment (start 143.8 84.728249) (end 143.8 85.175) (width 0.25) (layer "F.Cu") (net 2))
 (via (at 132 102) (size 0.8) (drill 0.4) (layers "F.Cu" "B.Cu") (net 2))
 (via (at 145.288 102.108) (size 0.8) (drill 0.4) (layers "F.Cu" "B.Cu") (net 2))
 (segment (start 135.55 81.9) (end 135.55 82.221368) (width 0.25) (layer "B.Cu") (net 2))
 (segment (start 132.406 98.799) (end 132.406 85.749) (width 0.25) (layer "B.Cu") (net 2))
 (segment (start 145.446 99.759) (end 145.288 99.917) (width 0.25) (layer "B.Cu") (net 2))
 (segment (start 135.55 82.221368) (end 133.446 84.325368) (width 0.25) (layer "B.Cu") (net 2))
 (segment (start 145.288 99.917) (end 145.288 102.108) (width 0.25) (layer "B.Cu") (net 2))
 (segment (start 132 102) (end 131.446 101.446) (width 0.25) (layer "B.Cu") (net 2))
 (segment (start 131.446 101.446) (end 131.446 99.759) (width 0.25) (layer "B.Cu") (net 2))
 (segment (start 131.446 99.759) (end 132.406 98.799) (width 0.25) (layer "B.Cu") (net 2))
 (segment (start 133.446 84.325368) (end 133.446 84.709) (width 0.25) (layer "B.Cu") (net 2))
 (segment (start 132.406 85.749) (end 133.446 84.709) (width 0.25) (layer "B.Cu") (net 2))
 (segment (start 131.5 90.05) (end 131.5 88.5565) (width 0.25) (layer "F.Cu") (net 6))
 (segment (start 144.45 92.202) (end 143.002 92.202) (width 0.25) (layer "F.Cu") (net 6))
 (segment (start 144.488 92.24) (end 144.45 92.202) (width 0.25) (layer "F.Cu") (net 6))
 (segment (start 142.24 91.44) (end 141.44 90.64) (width 0.25) (layer "F.Cu") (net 6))
 (segment (start 132.55 91.1) (end 131.5 90.05) (width 0.25) (layer "F.Cu") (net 6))
 (segment (start 131.5 88.5565) (end 132.0565 88) (width 0.25) (layer "F.Cu") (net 6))
 (segment (start 134.59 90.64) (end 136.906 90.64) (width 0.25) (layer "F.Cu") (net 6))
 (segment (start 134 90.05) (end 134.59 90.64) (width 0.25) (layer "F.Cu") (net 6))
 (segment (start 131.958 94.225) (end 131.958 93.030173) (width 0.25) (layer "F.Cu") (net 6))
 (segment (start 131.958 93.030173) (end 132.55 92.438173) (width 0.25) (layer "F.Cu") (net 6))
 (segment (start 132.55 92.438173) (end 132.55 91.1) (width 0.25) (layer "F.Cu") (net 6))
 (segment (start 136.5 89.5) (end 136.5 90.234) (width 0.25) (layer "F.Cu") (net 6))
 (segment (start 142.8 86.412) (end 142.8 85.175) (width 0.25) (layer "F.Cu") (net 6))
 (segment (start 141.44 90.64) (end 136.906 90.64) (width 0.25) (layer "F.Cu") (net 6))
 (segment (start 136.5 90.234) (end 136.906 90.64) (width 0.25) (layer "F.Cu") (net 6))
 (segment (start 145.406 92.24) (end 144.488 92.24) (width 0.25) (layer "F.Cu") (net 6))
 (segment (start 142.748 90.932) (end 142.24 91.44) (width 0.25) (layer "F.Cu") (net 6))
 (segment (start 143.51 87.122) (end 142.8 86.412) (width 0.25) (layer "F.Cu") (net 6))
 (segment (start 131.5 90.05) (end 134 90.05) (width 0.25) (layer "F.Cu") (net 6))
 (segment (start 143.002 92.202) (end 142.24 91.44) (width 0.25) (layer "F.Cu") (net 6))
 (via (at 143.51 87.122) (size 0.8) (drill 0.4) (layers "F.Cu" "B.Cu") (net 6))
 (via (at 136.5 89.5) (size 0.8) (drill 0.4) (layers "F.Cu" "B.Cu") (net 6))
 (via (at 142.748 90.932) (size 0.8) (drill 0.4) (layers "F.Cu" "B.Cu") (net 6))
 (segment (start 145.800305 96.775) (end 145.775 96.775) (width 0.25) (layer "B.Cu") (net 6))
 (segment (start 136.5 89) (end 136.5 89.5) (width 0.25) (layer "B.Cu") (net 6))
 (segment (start 136.5 88.956193) (end 136.5 89) (width 0.25) (layer "B.Cu") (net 6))
 (segment (start 139.446 84.709) (end 139.446 86.010193) (width 0.25) (layer "B.Cu") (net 6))
 (segment (start 139.446 83.896) (end 139.446 84.709) (width 0.25) (layer "B.Cu") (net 6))
 (segment (start 139.446 86.010193) (end 136.5 88.956193) (width 0.25) (layer "B.Cu") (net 6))
 (segment (start 145.775 96.775) (end 143.225 94.225) (width 0.25) (layer "B.Cu") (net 6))
 (segment (start 137.45 81.9) (end 139.446 83.896) (width 0.25) (layer "B.Cu") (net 6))
 (segment (start 150.5 96.96) (end 145.985305 96.96) (width 0.25) (layer "B.Cu") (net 6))
 (segment (start 145.985305 96.96) (end 145.800305 96.775) (width 0.25) (layer "B.Cu") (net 6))
 (segment (start 142.748 87.884) (end 142.748 90.932) (width 0.25) (layer "B.Cu") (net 6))
 (segment (start 143.51 87.122) (end 142.748 87.884) (width 0.25) (layer "B.Cu") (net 6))
 (segment (start 143.225 94.225) (end 143.225 91.409) (width 0.25) (layer "B.Cu") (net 6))
 (segment (start 143.225 91.409) (end 142.748 90.932) (width 0.25) (layer "B.Cu") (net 6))
 (segment (start 146.802 93.04) (end 145.406 93.04) (width 0.25) (layer "F.Cu") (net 8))
 (segment (start 147.447 92.395) (end 146.802 93.04) (width 0.25) (layer "F.Cu") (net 8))
 (segment (start 149.2 90.64) (end 150.5 89.34) (width 0.25) (layer "F.Cu") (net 11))
 (segment (start 145.406 90.64) (end 149.2 90.64) (width 0.25) (layer "F.Cu") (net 11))
 (segment (start 142.494 87.112695) (end 142.494 87.113402) (width 0.25) (layer "F.Cu") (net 17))
 (segment (start 138.356 96.603305) (end 138.356 97.69) (width 0.25) (layer "F.Cu") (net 17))
 (segment (start 141.8 86.418695) (end 142.494 87.112695) (width 0.25) (layer "F.Cu") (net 17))
 (segment (start 142.494 87.113402) (end 142.485402 87.122) (width 0.25) (layer "F.Cu") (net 17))
 (segment (start 141.8 85.175) (end 141.8 86.418695) (width 0.25) (layer "F.Cu") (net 17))
 (segment (start 141.467504 93.491801) (end 138.356 96.603305) (width 0.25) (layer "F.Cu") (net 17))
 (segment (start 141.467504 93.444307) (end 141.467504 93.491801) (width 0.25) (layer "F.Cu") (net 17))
 (via (at 142.485402 87.122) (size 0.8) (drill 0.4) (layers "F.Cu" "B.Cu") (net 17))
 (via (at 141.467504 93.444307) (size 0.8) (drill 0.4) (layers "F.Cu" "B.Cu") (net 17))
 (segment (start 142.298 87.309402) (end 142.485402 87.122) (width 0.25) (layer "B.Cu") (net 17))
 (segment (start 141.467504 93.444307) (end 141.467504 90.942496) (width 0.25) (layer "B.Cu") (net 17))
 (segment (start 142.298 90.112) (end 142.298 87.309402) (width 0.25) (layer "B.Cu") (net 17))
 (segment (start 141.467504 90.942496) (end 142.298 90.112) (width 0.25) (layer "B.Cu") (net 17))
 (segment (start 139.156 96.81) (end 141.478 94.488) (width 0.25) (layer "F.Cu") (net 18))
 (segment (start 140.8 85.175) (end 140.462 85.513) (width 0.25) (layer "F.Cu") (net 18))
 (segment (start 141.482653 94.492653) (end 141.491251 94.492653) (width 0.25) (layer "F.Cu") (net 18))
 (segment (start 141.478 94.488) (end 141.482653 94.492653) (width 0.25) (layer "F.Cu") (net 18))
 (segment (start 140.462 85.513) (end 140.462 87.63) (width 0.25) (layer "F.Cu") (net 18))
 (segment (start 139.156 97.69) (end 139.156 96.81) (width 0.25) (layer "F.Cu") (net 18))
 (via (at 141.491251 94.492653) (size 0.8) (drill 0.4) (layers "F.Cu" "B.Cu") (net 18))
 (via (at 140.462 87.63) (size 0.8) (drill 0.4) (layers "F.Cu" "B.Cu") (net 18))
 (segment (start 140.462 87.63) (end 140.462 93.463402) (width 0.25) (layer "B.Cu") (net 18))
 (segment (start 140.462 93.463402) (end 141.491251 94.492653) (width 0.25) (layer "B.Cu") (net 18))
 (segment (start 143.156 98.616315) (end 143.156 97.69) (width 0.2) (layer "F.Cu") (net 14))
 (segment (start 140.136 102.354) (end 140.136 101.636315) (width 0.2) (layer "F.Cu") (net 14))
 (segment (start 140.136 101.636315) (end 143.156 98.616315) (width 0.2) (layer "F.Cu") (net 14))
 (segment (start 143.956 97.69) (end 143.956 98.466315) (width 0.2) (layer "F.Cu") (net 15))
 (segment (start 143.956 98.466315) (end 140.786 101.636315) (width 0.2) (layer "F.Cu") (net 15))
 (segment (start 140.786 101.636315) (end 140.786 102.354) (width 0.2) (layer "F.Cu") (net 15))
 (segment (start 145.406 95.44) (end 146.6625 95.44) (width 0.25) (layer "F.Cu") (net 10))
 (segment (start 146.6625 95.44) (end 146.7225 95.5) (width 0.25) (layer "F.Cu") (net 10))
 (via (at 146.7225 95.5) (size 0.8) (drill 0.4) (layers "F.Cu" "B.Cu") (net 10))
 (segment (start 146.7225 95.5) (end 146.88 95.5) (width 0.25) (layer "B.Cu") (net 10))
 (segment (start 146.88 95.5) (end 150.5 91.88) (width 0.25) (layer "B.Cu") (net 10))
 (segment (start 145.406 96.24) (end 145.406 97.406) (width 0.25) (layer "F.Cu") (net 9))
 (segment (start 145.406 97.406) (end 145.5 97.5) (width 0.25) (layer "F.Cu") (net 9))
 (via (at 145.5 97.5) (size 0.8) (drill 0.4) (layers "F.Cu" "B.Cu") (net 9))
 (segment (start 148.5 97.5) (end 150.5 99.5) (width 0.25) (layer "B.Cu") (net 9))
 (segment (start 145.5 97.5) (end 148.5 97.5) (width 0.25) (layer "B.Cu") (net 9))
 (segment (start 151.675 87.975) (end 150.5 86.8) (width 0.25) (layer "F.Cu") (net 12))
 (segment (start 150.986701 90.515) (end 151.675 89.826701) (width 0.25) (layer "F.Cu") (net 12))
 (segment (start 151.675 89.826701) (end 151.675 87.975) (width 0.25) (layer "F.Cu") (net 12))
 (segment (start 149.278299 91.44) (end 150.203299 90.515) (width 0.25) (layer "F.Cu") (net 12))
 (segment (start 145.406 91.44) (end 149.278299 91.44) (width 0.25) (layer "F.Cu") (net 12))
 (segment (start 150.203299 90.515) (end 150.986701 90.515) (width 0.25) (layer "F.Cu") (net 12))
 (segment (start 139.13006 93.04) (end 139.238424 93.148364) (width 0.25) (layer "F.Cu") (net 26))
 (segment (start 136.906 93.04) (end 139.13006 93.04) (width 0.25) (layer "F.Cu") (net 26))
 (via (at 139.238424 93.148364) (size 0.8) (drill 0.4) (layers "F.Cu" "B.Cu") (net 26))
 (segment (start 139.238424 93.171576) (end 139.238424 93.148364) (width 0.25) (layer "B.Cu") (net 26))
 (segment (start 143.446 99.759) (end 143.446 97.472) (width 0.25) (layer "B.Cu") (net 26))
 (segment (start 139.192 93.218) (end 139.238424 93.171576) (width 0.25) (layer "B.Cu") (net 26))
 (segment (start 143.446 97.472) (end 139.192 93.218) (width 0.25) (layer "B.Cu") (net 26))
 (segment (start 138.544 93.84) (end 138.684 93.98) (width 0.25) (layer "F.Cu") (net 27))
 (segment (start 136.906 93.84) (end 138.544 93.84) (width 0.25) (layer "F.Cu") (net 27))
 (via (at 138.684 93.98) (size 0.8) (drill 0.4) (layers "F.Cu" "B.Cu") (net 27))
 (segment (start 141.446 96.742) (end 138.684 93.98) (width 0.25) (layer "B.Cu") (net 27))
 (segment (start 141.446 99.759) (end 141.446 96.742) (width 0.25) (layer "B.Cu") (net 27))
 (segment (start 137.956 94.64) (end 138.43 95.114) (width 0.25) (layer "F.Cu") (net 28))
 (segment (start 136.906 94.64) (end 137.956 94.64) (width 0.25) (layer "F.Cu") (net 28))
 (segment (start 138.43 95.114) (end 138.43 95.504) (width 0.25) (layer "F.Cu") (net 28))
 (via (at 138.43 95.504) (size 0.8) (drill 0.4) (layers "F.Cu" "B.Cu") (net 28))
 (segment (start 138.43 98.743) (end 138.43 95.504) (width 0.25) (layer "B.Cu") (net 28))
 (segment (start 139.446 99.759) (end 138.43 98.743) (width 0.25) (layer "B.Cu") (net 28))
 (segment (start 135.382 95.758) (end 135.509 95.631) (width 0.25) (layer "F.Cu") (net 29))
 (segment (start 135.7 95.44) (end 135.509 95.631) (width 0.25) (layer "F.Cu") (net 29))
 (segment (start 136.906 95.44) (end 135.7 95.44) (width 0.25) (layer "F.Cu") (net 29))
 (via (at 135.509 95.631) (size 0.8) (drill 0.4) (layers "F.Cu" "B.Cu") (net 29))
 (segment (start 135.509 95.631) (end 137.446 97.568) (width 0.25) (layer "B.Cu") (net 29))
 (segment (start 137.446 97.568) (end 137.446 99.759) (width 0.25) (layer "B.Cu") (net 29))
 (segment (start 136.424 96.24) (end 135.382 97.282) (width 0.25) (layer "F.Cu") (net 30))
 (segment (start 136.906 96.24) (end 136.424 96.24) (width 0.25) (layer "F.Cu") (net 30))
 (via (at 135.382 97.282) (size 0.8) (drill 0.4) (layers "F.Cu" "B.Cu") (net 30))
 (segment (start 135.382 99.695) (end 135.446 99.759) (width 0.25) (layer "B.Cu") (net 30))
 (segment (start 135.382 97.282) (end 135.382 99.695) (width 0.25) (layer "B.Cu") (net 30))
 (segment (start 131.572 84.583) (end 131.446 84.709) (width 0.25) (layer "B.Cu") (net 3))
 (segment (start 131.572 81.28) (end 131.572 84.583) (width 0.25) (layer "B.Cu") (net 3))
 (segment (start 141.556 89.19) (end 141.556 87.2) (width 0.25) (layer "F.Cu") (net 22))
 (segment (start 141.556 87.2) (end 141.478 87.122) (width 0.25) (layer "F.Cu") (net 22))
 (via (at 141.478 87.122) (size 0.8) (drill 0.4) (layers "F.Cu" "B.Cu") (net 22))
 (segment (start 141.446 87.09) (end 141.478 87.122) (width 0.25) (layer "B.Cu") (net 22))
 (segment (start 141.446 84.709) (end 141.446 87.09) (width 0.25) (layer "B.Cu") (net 22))
 (segment (start 135.1 81) (end 137 81) (width 0.25) (layer "F.Cu") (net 4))
 (segment (start 135.76 92.24) (end 135.5 92.5) (width 0.25) (layer "F.Cu") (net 7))
 (segment (start 134.8815 89) (end 133.8815 88) (width 0.25) (layer "F.Cu") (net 7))
 (segment (start 136.906 92.24) (end 135.76 92.24) (width 0.25) (layer "F.Cu") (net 7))
 (segment (start 135.5 89) (end 134.8815 89) (width 0.25) (layer "F.Cu") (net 7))
 (via (at 135.5 89) (size 0.8) (drill 0.4) (layers "F.Cu" "B.Cu") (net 7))
 (via (at 135.5 92.5) (size 0.8) (drill 0.4) (layers "F.Cu" "B.Cu") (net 7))
 (segment (start 135.5 92.5) (end 135.5 89) (width 0.25) (layer "B.Cu") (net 7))
 (segment (start 135.5 85) (end 138.356 87.856) (width 0.25) (layer "F.Cu") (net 5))
 (segment (start 135.5 83.225) (end 135.5 85) (width 0.25) (layer "F.Cu") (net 5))
 (segment (start 135.1 82.825) (end 135.5 83.225) (width 0.25) (layer "F.Cu") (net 5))
 (segment (start 138.356 87.856) (end 138.356 89.19) (width 0.25) (layer "F.Cu") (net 5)))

